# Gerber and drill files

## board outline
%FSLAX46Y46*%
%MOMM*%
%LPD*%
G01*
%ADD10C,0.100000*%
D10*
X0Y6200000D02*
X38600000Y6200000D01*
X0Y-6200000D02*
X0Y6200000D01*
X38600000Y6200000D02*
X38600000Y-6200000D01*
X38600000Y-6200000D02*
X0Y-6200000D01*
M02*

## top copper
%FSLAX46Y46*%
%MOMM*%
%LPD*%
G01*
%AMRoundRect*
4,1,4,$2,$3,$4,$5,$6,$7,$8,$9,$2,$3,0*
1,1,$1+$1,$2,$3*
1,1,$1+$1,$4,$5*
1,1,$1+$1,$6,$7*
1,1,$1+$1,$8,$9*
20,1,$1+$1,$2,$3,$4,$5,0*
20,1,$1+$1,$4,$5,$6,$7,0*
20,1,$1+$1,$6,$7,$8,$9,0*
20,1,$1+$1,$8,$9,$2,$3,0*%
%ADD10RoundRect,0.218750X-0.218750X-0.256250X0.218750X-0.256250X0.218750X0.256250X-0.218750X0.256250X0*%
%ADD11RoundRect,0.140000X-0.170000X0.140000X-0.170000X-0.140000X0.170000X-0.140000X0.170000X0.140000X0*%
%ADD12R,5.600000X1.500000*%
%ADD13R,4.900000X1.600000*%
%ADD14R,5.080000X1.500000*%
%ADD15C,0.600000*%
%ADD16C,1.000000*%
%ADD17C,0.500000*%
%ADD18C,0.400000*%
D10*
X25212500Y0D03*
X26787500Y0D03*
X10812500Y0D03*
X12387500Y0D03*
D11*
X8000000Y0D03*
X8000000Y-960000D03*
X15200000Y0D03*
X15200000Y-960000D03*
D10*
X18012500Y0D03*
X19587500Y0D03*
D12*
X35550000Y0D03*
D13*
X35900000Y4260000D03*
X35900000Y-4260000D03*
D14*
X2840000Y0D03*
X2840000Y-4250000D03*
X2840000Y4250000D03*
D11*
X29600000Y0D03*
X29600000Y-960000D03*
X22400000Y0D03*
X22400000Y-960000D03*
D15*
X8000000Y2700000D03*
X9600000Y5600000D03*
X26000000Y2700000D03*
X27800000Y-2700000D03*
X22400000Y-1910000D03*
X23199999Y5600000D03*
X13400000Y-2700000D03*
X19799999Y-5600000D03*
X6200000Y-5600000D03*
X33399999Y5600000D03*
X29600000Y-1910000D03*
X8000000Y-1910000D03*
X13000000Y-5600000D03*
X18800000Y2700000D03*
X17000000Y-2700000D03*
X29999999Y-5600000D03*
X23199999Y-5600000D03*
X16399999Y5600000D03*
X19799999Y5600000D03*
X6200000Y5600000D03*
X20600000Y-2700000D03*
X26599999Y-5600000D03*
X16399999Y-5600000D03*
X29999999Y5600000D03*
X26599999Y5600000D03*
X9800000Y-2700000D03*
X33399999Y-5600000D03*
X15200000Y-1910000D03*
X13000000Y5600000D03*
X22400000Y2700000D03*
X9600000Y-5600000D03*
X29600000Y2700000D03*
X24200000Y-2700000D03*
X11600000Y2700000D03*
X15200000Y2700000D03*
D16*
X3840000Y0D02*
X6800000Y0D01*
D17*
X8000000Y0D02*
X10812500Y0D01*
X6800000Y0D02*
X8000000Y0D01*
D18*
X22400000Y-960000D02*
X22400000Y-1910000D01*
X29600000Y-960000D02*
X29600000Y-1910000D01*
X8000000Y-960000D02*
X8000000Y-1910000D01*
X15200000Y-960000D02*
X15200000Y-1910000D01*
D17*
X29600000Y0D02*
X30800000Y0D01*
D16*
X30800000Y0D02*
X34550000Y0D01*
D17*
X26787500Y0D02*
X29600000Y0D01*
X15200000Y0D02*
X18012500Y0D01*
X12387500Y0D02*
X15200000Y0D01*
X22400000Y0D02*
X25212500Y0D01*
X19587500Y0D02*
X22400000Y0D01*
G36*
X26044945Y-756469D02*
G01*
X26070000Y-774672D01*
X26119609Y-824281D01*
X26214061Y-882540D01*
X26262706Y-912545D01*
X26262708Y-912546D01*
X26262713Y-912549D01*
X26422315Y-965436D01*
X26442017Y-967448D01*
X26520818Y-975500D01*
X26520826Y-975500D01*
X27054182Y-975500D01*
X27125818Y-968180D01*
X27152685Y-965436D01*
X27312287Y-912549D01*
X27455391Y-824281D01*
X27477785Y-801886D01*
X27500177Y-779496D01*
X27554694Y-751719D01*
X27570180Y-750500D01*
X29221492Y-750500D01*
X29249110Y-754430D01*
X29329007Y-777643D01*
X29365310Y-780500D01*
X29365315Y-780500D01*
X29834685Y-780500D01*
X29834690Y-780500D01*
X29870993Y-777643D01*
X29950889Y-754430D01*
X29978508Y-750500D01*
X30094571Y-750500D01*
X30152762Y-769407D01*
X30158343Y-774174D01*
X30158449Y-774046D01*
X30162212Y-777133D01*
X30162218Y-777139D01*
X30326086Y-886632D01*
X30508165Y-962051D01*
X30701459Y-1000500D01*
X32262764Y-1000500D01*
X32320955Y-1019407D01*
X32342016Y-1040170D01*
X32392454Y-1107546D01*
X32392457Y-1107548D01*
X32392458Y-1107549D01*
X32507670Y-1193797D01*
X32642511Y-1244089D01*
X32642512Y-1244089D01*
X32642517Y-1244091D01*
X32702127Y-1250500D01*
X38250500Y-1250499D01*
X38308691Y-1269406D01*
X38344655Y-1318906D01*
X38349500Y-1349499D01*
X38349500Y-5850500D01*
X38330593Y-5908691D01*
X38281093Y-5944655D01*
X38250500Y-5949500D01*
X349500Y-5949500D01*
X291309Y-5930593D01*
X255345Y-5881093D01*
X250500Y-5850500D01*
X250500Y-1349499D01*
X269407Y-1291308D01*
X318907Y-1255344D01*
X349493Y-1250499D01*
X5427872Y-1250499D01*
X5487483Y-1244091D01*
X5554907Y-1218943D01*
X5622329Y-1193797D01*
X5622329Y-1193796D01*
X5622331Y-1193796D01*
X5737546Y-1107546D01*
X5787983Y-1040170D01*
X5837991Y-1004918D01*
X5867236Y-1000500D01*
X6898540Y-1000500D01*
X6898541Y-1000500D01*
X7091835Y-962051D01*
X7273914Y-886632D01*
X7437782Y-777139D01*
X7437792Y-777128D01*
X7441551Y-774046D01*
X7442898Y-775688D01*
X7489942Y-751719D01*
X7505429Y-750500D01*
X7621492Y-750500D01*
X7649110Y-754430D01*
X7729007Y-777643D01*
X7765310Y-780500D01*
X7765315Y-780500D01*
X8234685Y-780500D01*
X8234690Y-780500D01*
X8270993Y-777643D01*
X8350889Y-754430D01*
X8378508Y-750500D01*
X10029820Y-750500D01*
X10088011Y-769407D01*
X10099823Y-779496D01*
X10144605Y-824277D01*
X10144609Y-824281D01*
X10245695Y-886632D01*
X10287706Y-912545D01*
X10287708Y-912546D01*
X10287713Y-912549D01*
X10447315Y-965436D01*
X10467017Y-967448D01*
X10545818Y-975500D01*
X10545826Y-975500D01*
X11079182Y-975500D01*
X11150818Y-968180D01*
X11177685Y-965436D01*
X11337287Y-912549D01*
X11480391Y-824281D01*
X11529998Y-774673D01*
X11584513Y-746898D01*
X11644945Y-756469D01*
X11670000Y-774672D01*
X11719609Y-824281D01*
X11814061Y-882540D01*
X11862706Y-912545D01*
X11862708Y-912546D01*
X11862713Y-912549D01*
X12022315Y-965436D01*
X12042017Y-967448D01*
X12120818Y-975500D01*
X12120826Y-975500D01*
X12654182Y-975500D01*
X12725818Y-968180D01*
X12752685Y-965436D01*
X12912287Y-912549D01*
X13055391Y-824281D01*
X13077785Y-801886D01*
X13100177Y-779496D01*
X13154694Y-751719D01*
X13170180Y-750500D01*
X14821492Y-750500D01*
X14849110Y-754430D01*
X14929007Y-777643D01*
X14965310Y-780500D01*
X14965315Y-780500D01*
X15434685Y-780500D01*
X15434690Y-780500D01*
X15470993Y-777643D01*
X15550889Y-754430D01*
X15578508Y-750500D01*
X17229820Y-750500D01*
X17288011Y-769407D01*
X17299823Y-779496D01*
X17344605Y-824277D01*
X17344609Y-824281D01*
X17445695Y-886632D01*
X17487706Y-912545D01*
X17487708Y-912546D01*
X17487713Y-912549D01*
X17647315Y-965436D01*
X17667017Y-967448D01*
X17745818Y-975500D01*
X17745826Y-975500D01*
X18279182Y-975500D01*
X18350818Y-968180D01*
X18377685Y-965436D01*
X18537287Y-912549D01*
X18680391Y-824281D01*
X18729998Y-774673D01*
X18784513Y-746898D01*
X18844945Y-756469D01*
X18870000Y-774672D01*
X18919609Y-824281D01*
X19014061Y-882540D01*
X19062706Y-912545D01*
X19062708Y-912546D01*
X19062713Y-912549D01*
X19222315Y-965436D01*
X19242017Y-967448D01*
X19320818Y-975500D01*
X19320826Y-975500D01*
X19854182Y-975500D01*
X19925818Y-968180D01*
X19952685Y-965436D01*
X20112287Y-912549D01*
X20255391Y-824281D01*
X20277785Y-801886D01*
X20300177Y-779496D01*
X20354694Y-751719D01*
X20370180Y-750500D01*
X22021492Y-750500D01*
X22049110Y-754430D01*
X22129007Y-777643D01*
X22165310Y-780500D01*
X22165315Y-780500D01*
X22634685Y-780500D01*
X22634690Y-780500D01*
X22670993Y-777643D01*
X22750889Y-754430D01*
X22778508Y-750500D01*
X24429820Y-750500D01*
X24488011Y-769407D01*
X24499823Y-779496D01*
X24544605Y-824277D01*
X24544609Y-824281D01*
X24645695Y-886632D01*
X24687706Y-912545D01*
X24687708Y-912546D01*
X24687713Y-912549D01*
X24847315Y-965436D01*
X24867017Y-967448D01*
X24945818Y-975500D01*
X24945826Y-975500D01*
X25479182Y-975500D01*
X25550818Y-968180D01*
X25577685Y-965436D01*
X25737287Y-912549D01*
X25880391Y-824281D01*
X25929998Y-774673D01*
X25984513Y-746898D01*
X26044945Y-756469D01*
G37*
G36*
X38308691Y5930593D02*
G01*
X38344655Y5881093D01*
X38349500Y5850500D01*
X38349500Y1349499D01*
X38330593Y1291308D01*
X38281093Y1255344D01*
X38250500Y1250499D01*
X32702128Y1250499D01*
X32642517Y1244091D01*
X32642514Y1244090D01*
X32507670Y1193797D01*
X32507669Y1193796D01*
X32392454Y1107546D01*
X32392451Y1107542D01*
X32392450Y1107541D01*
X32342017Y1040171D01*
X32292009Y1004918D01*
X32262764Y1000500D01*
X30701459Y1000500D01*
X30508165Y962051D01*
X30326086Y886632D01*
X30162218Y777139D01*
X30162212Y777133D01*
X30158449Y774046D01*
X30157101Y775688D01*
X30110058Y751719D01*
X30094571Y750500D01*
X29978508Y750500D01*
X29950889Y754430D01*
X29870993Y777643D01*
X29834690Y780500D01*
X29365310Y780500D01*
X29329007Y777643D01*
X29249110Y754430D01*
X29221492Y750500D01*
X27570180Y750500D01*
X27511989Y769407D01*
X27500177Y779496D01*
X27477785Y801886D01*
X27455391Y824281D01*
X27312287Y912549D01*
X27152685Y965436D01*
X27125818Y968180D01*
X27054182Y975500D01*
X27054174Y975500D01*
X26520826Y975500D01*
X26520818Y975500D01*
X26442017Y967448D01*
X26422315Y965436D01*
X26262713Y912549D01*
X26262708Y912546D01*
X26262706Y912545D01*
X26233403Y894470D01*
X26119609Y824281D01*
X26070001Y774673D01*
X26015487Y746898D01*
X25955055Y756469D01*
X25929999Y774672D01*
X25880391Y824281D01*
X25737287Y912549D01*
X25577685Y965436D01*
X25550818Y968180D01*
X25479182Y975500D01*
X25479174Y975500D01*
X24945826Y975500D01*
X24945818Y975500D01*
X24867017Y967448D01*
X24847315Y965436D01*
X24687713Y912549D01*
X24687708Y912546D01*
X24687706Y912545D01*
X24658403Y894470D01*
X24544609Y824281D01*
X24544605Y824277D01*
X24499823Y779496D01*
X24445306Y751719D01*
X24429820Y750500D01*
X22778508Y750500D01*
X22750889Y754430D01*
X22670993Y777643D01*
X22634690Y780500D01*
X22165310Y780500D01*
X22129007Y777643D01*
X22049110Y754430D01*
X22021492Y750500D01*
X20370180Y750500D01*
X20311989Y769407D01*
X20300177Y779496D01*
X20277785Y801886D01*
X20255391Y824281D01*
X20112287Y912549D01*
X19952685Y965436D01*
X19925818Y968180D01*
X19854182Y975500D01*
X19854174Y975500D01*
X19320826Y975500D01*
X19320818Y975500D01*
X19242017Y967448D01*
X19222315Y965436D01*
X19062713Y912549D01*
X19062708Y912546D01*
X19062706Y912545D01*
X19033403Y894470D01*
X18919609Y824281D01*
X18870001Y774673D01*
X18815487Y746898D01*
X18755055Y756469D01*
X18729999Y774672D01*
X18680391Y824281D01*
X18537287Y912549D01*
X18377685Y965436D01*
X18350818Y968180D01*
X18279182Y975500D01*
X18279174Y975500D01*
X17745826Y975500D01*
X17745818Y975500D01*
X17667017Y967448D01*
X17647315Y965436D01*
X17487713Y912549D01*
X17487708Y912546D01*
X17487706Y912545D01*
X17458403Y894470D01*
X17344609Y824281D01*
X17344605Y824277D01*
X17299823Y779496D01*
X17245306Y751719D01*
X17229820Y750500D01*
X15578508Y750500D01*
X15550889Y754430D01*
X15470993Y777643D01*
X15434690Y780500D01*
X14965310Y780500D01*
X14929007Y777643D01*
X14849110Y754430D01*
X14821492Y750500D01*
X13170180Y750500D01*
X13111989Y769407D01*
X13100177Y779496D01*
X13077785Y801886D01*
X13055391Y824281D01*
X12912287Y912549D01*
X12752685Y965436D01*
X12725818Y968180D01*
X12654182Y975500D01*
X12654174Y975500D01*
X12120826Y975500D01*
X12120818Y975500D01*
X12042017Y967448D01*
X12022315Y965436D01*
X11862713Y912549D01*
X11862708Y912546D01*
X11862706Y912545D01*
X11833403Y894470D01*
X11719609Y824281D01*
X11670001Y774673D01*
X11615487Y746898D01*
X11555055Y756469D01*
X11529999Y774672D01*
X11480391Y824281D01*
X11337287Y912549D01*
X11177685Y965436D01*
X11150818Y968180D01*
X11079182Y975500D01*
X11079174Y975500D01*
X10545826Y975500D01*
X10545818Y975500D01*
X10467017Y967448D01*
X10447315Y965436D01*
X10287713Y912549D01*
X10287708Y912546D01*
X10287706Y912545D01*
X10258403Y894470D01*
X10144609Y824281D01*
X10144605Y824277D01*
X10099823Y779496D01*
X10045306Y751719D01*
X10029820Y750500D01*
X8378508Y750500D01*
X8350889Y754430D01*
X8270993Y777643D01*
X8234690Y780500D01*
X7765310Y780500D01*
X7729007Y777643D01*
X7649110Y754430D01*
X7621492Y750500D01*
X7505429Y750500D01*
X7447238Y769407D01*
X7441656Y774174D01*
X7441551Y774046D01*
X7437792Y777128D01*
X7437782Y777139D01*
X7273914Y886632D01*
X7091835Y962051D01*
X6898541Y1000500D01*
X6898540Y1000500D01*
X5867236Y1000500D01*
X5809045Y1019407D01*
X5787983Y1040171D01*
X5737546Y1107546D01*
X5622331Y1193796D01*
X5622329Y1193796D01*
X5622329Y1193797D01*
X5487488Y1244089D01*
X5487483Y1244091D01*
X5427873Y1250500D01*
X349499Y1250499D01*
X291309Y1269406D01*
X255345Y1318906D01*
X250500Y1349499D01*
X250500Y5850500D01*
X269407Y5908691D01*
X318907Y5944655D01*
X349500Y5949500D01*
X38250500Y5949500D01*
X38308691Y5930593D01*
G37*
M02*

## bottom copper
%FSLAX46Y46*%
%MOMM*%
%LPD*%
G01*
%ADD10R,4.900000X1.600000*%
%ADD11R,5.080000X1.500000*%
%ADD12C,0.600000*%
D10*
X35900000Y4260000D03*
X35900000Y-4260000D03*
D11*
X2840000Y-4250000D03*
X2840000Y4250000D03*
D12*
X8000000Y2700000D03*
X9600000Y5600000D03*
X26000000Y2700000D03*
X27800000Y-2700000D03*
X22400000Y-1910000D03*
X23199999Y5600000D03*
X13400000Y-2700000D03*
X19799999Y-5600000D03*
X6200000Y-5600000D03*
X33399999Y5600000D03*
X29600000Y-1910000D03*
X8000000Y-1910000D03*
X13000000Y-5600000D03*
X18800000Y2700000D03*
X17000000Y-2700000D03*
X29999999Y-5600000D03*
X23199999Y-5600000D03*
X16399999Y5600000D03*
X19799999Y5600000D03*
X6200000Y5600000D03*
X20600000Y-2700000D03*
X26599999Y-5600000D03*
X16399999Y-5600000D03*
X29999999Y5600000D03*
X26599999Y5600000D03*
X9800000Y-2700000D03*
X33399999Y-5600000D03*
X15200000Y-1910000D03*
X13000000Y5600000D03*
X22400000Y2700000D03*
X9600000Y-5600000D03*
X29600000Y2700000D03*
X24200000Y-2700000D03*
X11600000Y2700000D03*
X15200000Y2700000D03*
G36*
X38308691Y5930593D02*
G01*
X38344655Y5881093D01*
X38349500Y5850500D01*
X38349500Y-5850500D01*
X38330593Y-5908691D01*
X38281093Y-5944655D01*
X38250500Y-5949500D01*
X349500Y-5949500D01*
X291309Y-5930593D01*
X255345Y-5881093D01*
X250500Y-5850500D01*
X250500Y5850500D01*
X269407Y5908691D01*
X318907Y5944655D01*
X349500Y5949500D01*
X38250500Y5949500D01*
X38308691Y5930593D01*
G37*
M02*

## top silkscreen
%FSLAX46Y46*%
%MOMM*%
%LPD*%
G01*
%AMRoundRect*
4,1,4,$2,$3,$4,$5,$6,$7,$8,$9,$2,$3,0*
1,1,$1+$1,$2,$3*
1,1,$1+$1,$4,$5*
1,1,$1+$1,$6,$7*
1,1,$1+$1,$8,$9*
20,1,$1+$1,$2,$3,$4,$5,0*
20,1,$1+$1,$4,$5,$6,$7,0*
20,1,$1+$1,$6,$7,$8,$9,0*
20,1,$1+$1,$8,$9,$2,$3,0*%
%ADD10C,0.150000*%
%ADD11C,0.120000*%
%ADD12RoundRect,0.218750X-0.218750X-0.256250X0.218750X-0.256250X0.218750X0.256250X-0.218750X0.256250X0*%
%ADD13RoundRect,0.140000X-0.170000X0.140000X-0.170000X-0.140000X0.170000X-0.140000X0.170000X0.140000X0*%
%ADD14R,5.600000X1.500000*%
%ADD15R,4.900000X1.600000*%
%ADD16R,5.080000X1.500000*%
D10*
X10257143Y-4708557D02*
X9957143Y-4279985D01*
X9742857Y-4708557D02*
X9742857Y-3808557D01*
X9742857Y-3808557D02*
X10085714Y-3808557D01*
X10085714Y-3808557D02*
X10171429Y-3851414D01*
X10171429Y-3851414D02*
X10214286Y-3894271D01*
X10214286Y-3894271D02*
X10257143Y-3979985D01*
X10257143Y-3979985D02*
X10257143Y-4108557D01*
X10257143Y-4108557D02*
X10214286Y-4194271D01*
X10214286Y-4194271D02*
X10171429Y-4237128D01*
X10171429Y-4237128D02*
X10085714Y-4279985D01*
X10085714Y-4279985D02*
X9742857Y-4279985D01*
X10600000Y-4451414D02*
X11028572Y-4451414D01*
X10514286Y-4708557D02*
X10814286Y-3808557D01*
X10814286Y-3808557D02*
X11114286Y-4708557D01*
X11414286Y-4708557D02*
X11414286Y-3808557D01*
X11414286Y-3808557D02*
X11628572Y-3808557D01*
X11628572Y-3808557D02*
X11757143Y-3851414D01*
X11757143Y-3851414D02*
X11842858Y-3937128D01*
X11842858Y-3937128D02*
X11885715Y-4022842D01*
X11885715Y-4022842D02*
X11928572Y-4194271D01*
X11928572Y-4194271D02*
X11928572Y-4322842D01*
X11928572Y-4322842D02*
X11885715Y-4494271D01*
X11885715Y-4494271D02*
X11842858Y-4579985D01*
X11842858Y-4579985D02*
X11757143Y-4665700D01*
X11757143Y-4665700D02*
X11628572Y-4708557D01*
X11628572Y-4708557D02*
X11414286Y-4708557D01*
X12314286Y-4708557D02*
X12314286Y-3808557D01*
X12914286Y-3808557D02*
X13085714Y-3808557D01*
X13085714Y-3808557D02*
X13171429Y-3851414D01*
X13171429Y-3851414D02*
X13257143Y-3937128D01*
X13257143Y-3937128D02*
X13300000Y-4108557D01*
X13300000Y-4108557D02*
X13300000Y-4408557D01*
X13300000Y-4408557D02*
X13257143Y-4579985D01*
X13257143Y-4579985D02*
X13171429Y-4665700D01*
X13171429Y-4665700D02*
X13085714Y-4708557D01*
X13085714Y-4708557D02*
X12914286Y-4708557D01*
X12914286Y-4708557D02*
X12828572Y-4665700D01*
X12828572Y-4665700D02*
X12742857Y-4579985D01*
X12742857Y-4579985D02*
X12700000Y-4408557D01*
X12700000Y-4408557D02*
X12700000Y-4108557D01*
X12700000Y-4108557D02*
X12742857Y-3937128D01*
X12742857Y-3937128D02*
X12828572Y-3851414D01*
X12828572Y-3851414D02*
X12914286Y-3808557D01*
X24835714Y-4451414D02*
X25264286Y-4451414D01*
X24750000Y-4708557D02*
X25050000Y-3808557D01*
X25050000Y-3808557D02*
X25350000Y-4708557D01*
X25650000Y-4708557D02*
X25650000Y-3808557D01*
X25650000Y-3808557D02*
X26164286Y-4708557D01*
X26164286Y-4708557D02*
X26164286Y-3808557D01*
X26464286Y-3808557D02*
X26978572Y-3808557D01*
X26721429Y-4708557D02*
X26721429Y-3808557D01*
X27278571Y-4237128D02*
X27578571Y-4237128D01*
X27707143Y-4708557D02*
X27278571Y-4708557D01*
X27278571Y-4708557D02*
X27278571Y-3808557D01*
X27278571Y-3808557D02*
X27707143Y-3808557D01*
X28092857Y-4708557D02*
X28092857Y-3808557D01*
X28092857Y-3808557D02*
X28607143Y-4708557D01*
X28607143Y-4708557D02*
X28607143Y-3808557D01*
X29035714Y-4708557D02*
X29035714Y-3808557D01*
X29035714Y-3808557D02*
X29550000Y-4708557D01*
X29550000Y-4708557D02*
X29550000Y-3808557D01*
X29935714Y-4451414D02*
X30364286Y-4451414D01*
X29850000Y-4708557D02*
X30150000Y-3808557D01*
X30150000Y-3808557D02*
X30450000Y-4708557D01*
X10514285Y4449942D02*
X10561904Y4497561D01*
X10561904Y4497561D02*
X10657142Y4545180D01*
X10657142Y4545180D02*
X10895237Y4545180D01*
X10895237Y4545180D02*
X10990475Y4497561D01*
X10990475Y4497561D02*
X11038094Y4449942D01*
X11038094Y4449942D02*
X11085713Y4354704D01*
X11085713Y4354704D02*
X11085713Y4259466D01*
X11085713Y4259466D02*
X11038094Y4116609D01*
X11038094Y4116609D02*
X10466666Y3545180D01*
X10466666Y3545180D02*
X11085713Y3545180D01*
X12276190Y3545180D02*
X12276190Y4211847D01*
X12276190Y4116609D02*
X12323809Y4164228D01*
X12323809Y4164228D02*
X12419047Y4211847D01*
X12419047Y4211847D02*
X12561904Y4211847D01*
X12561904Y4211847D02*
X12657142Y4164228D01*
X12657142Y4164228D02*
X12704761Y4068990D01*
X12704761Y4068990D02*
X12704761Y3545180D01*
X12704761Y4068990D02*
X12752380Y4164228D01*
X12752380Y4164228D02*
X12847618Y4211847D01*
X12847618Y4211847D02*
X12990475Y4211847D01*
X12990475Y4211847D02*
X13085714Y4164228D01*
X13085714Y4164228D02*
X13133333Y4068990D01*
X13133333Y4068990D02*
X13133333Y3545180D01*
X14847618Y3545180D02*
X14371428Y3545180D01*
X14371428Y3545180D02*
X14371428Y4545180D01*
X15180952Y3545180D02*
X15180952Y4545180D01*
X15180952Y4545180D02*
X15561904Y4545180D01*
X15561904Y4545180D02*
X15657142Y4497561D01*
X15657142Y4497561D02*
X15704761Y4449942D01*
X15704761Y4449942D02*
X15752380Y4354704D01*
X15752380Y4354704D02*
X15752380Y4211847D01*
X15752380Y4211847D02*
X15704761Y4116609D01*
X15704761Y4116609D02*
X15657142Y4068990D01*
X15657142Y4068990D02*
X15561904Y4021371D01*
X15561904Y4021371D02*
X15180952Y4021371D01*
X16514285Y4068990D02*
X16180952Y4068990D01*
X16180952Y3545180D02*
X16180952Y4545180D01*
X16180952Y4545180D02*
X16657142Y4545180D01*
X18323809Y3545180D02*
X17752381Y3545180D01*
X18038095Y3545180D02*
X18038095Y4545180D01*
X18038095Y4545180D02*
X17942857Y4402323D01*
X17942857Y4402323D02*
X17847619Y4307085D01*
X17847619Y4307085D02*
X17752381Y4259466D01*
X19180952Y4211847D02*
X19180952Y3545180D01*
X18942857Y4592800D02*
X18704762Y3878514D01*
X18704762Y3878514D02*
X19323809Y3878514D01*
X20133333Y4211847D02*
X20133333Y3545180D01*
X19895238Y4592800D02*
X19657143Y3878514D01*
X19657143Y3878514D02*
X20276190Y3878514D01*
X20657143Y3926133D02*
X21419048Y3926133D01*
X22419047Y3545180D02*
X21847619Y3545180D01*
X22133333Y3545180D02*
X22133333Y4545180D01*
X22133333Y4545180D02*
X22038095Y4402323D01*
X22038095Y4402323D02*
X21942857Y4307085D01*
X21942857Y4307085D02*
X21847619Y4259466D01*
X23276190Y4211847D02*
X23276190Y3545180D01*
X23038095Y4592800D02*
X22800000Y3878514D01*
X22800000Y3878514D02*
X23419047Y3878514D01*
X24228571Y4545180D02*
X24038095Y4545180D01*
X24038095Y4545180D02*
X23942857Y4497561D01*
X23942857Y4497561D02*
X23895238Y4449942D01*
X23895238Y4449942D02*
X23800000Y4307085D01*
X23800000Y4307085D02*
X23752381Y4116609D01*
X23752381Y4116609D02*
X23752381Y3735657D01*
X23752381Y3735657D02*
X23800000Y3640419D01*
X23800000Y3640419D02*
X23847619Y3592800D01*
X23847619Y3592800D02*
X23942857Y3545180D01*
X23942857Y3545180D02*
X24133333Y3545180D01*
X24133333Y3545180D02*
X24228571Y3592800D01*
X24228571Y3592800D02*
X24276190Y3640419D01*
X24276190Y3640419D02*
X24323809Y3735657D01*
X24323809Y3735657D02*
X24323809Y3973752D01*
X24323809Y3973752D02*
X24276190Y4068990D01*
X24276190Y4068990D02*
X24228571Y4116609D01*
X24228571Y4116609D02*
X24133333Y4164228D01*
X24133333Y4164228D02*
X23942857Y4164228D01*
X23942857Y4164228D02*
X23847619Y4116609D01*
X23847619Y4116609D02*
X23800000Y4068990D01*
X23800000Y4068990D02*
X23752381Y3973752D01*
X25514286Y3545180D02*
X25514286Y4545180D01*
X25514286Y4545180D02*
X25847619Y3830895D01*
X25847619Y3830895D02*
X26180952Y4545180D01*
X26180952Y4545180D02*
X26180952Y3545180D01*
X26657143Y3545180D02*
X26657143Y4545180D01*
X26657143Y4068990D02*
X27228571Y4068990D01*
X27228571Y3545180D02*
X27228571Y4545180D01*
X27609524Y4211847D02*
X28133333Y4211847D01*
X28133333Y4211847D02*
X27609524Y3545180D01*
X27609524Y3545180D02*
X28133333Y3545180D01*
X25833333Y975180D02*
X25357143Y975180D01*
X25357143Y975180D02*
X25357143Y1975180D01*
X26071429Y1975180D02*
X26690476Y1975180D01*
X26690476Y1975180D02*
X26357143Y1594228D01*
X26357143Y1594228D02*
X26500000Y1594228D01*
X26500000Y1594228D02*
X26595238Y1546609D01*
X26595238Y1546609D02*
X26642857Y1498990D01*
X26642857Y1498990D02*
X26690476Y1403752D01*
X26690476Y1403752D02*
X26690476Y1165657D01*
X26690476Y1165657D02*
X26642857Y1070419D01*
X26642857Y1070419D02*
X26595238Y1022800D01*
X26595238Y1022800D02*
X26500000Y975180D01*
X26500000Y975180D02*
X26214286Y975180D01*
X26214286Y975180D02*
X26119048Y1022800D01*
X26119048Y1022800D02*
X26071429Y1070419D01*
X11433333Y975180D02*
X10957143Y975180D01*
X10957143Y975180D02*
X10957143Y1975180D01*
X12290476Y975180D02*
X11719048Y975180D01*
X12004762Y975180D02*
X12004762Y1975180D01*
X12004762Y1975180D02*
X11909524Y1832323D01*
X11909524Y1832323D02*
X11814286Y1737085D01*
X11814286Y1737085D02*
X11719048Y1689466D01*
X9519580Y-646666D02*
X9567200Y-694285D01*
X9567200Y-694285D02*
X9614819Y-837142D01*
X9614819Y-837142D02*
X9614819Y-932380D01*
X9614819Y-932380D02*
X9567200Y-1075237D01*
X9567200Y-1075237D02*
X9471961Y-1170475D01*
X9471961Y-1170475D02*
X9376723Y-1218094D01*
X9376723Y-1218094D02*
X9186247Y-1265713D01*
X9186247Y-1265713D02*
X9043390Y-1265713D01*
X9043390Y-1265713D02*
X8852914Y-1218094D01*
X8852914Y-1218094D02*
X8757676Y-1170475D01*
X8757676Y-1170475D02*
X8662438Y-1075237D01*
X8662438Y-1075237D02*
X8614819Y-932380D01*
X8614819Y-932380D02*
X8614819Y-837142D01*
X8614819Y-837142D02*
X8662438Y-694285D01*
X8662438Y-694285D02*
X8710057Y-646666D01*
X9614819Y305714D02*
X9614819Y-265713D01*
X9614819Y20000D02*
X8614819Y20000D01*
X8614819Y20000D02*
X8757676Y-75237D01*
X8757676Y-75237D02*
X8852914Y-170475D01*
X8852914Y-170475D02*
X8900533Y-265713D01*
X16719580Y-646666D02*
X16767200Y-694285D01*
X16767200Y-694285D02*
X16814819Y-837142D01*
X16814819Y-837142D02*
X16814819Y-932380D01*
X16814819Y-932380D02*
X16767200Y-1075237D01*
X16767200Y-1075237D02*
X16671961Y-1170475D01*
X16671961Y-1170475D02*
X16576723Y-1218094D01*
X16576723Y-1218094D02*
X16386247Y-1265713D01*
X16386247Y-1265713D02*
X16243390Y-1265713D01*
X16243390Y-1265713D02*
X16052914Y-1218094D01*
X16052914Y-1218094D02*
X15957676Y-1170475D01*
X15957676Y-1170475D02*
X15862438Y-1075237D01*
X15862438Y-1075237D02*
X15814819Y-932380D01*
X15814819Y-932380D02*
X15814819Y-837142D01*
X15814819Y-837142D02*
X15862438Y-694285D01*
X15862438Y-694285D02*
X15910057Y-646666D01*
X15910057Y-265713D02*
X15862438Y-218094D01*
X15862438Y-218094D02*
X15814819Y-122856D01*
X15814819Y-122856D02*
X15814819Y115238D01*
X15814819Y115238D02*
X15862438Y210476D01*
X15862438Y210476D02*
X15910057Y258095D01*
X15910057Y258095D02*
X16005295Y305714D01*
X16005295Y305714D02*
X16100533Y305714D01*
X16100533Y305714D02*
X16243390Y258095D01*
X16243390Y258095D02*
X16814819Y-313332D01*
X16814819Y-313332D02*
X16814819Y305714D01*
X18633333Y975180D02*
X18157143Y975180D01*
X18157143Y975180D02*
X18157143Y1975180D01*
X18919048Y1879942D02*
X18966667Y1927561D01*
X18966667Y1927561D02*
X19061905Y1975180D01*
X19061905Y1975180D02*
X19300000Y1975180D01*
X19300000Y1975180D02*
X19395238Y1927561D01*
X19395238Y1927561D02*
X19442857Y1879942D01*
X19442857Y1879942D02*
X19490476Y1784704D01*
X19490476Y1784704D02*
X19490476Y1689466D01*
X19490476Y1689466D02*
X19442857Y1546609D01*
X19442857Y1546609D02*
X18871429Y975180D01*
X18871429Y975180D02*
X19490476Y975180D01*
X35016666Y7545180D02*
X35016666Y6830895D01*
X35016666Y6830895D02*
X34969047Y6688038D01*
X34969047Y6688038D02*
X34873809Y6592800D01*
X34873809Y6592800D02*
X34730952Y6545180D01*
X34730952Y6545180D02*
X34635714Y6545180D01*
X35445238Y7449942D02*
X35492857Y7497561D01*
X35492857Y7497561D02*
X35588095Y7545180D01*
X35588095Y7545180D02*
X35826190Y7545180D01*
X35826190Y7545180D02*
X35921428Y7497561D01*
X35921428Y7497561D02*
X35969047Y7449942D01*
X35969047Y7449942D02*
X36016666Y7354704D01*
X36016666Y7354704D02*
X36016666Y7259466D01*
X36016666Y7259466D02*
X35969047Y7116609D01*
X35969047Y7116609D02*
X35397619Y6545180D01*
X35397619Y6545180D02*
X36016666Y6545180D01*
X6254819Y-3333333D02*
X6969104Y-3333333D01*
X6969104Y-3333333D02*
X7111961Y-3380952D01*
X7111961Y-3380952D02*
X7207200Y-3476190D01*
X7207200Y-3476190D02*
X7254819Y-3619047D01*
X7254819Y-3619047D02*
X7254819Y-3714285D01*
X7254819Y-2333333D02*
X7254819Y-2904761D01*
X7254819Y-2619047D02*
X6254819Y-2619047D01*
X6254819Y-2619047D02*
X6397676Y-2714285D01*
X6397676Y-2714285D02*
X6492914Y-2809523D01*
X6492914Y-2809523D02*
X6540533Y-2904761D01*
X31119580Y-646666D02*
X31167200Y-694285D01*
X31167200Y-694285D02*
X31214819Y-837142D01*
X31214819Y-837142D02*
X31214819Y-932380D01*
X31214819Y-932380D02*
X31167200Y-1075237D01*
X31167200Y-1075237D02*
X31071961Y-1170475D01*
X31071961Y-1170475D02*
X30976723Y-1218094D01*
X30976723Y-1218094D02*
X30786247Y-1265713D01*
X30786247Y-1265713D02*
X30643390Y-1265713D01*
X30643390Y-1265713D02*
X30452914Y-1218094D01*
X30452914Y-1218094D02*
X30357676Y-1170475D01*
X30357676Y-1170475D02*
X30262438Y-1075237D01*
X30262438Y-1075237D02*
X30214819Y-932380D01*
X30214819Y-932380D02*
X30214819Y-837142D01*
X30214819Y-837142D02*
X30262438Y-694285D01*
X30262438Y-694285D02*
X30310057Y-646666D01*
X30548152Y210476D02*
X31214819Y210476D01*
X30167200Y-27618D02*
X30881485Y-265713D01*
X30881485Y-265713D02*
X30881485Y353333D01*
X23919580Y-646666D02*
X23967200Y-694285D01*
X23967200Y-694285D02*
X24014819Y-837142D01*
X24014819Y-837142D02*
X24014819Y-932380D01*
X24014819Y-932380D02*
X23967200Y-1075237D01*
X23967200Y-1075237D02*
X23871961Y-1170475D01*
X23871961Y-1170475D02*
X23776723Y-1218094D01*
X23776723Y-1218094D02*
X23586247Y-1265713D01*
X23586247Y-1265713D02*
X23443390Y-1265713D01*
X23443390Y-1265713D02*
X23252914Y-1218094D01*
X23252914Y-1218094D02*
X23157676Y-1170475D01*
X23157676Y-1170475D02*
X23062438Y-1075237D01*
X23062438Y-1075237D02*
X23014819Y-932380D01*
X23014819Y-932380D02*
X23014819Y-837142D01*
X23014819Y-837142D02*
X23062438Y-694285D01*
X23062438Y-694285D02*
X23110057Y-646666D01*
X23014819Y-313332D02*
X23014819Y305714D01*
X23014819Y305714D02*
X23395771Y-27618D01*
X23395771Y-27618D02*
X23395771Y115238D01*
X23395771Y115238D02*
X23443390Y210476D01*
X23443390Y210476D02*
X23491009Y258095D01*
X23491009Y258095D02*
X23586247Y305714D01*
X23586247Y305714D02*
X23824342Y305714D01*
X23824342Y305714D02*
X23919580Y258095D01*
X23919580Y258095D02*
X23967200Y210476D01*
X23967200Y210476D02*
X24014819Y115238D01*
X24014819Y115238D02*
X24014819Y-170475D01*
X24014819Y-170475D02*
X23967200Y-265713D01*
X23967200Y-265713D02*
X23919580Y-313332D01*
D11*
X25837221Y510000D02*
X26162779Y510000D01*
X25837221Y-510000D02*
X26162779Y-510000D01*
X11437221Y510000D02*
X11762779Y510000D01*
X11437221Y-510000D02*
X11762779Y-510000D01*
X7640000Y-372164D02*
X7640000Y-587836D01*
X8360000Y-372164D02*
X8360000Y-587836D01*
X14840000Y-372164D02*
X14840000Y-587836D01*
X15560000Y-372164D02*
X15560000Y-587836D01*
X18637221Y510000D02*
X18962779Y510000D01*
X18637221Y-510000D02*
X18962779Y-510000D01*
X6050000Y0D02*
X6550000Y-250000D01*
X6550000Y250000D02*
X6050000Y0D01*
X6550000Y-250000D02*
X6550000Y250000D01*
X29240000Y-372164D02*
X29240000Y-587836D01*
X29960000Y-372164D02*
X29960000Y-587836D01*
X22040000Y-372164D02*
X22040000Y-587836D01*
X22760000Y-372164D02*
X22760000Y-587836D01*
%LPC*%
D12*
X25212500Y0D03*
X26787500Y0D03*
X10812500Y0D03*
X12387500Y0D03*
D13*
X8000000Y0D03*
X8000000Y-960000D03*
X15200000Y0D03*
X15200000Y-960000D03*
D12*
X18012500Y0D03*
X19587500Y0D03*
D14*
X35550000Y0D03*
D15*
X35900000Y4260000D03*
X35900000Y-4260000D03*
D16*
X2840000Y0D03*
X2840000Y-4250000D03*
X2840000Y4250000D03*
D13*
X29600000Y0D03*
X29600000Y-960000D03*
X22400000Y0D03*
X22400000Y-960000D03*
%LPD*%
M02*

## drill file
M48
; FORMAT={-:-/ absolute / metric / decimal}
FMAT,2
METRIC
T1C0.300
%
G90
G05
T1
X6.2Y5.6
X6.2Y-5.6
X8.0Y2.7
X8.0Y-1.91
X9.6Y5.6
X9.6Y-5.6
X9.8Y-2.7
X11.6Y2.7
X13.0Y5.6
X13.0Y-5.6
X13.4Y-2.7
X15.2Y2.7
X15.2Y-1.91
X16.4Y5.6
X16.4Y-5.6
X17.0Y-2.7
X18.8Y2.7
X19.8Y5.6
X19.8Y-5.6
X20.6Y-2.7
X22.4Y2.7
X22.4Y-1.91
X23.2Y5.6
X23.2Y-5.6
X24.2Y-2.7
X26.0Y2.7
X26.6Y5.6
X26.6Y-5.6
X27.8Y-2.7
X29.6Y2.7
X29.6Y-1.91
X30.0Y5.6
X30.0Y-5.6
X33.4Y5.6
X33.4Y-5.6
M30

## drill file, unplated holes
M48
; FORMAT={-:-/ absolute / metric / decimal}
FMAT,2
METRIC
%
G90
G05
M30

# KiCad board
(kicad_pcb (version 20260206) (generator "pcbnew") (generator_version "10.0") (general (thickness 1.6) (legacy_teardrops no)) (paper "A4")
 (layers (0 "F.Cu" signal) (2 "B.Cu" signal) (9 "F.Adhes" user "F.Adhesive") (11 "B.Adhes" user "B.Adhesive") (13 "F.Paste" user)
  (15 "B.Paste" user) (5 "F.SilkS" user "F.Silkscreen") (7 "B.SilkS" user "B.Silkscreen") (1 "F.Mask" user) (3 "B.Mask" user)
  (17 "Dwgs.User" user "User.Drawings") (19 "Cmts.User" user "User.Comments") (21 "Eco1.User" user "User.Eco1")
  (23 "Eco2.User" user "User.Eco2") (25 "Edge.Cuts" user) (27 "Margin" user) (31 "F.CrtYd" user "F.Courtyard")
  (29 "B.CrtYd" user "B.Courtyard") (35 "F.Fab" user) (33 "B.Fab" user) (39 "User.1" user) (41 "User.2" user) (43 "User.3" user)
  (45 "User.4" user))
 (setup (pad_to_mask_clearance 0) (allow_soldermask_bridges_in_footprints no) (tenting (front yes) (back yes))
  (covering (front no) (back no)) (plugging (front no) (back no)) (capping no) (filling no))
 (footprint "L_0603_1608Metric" (layer "F.Cu") (at 26 0)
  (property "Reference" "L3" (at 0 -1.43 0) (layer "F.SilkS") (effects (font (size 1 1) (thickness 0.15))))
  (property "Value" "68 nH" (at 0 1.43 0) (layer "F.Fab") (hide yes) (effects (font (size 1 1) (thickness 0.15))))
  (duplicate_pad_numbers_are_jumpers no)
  (fp_line (start -0.162779 -0.51) (end 0.162779 -0.51) (stroke (width 0.12) (type solid)) (layer "F.SilkS"))
  (fp_line (start -0.162779 0.51) (end 0.162779 0.51) (stroke (width 0.12) (type solid)) (layer "F.SilkS"))
  (pad "1" smd roundrect (at -0.7875 0) (size 0.875 0.95) (layers "F.Cu" "F.Mask" "F.Paste") (roundrect_rratio 0.25) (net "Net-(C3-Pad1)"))
  (pad "2" smd roundrect (at 0.7875 0) (size 0.875 0.95) (layers "F.Cu" "F.Mask" "F.Paste") (roundrect_rratio 0.25) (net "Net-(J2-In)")))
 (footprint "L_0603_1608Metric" (layer "F.Cu") (at 11.6 0)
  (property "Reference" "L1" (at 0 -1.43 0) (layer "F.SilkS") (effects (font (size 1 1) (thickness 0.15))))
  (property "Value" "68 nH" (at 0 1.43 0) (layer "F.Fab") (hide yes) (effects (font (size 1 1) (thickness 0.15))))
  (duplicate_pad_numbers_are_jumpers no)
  (fp_line (start -0.162779 -0.51) (end 0.162779 -0.51) (stroke (width 0.12) (type solid)) (layer "F.SilkS"))
  (fp_line (start -0.162779 0.51) (end 0.162779 0.51) (stroke (width 0.12) (type solid)) (layer "F.SilkS"))
  (pad "1" smd roundrect (at -0.7875 0) (size 0.875 0.95) (layers "F.Cu" "F.Mask" "F.Paste") (roundrect_rratio 0.25) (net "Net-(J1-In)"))
  (pad "2" smd roundrect (at 0.7875 0) (size 0.875 0.95) (layers "F.Cu" "F.Mask" "F.Paste") (roundrect_rratio 0.25) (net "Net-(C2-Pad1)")))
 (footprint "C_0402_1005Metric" (layer "F.Cu") (at 8 0.48 -90)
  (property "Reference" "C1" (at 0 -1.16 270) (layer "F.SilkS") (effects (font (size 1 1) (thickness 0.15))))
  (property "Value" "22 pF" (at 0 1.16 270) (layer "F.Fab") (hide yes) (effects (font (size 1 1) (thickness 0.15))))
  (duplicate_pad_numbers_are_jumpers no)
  (fp_line (start -0.107836 0.36) (end 0.107836 0.36) (stroke (width 0.12) (type solid)) (layer "F.SilkS"))
  (fp_line (start -0.107836 -0.36) (end 0.107836 -0.36) (stroke (width 0.12) (type solid)) (layer "F.SilkS"))
  (pad "1" smd roundrect (at -0.48 0 270) (size 0.56 0.62) (layers "F.Cu" "F.Mask" "F.Paste") (roundrect_rratio 0.25) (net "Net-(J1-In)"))
  (pad "2" smd roundrect (at 0.48 0 270) (size 0.56 0.62) (layers "F.Cu" "F.Mask" "F.Paste") (roundrect_rratio 0.25) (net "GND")
   (zone_connect 2)))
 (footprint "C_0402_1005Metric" (layer "F.Cu") (at 15.2 0.48 -90)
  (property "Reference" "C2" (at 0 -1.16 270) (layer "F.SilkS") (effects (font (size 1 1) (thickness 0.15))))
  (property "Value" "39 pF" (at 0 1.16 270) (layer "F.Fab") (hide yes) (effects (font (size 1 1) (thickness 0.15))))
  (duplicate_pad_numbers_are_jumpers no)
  (fp_line (start -0.107836 0.36) (end 0.107836 0.36) (stroke (width 0.12) (type solid)) (layer "F.SilkS"))
  (fp_line (start -0.107836 -0.36) (end 0.107836 -0.36) (stroke (width 0.12) (type solid)) (layer "F.SilkS"))
  (pad "1" smd roundrect (at -0.48 0 270) (size 0.56 0.62) (layers "F.Cu" "F.Mask" "F.Paste") (roundrect_rratio 0.25) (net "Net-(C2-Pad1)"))
  (pad "2" smd roundrect (at 0.48 0 270) (size 0.56 0.62) (layers "F.Cu" "F.Mask" "F.Paste") (roundrect_rratio 0.25) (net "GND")
   (zone_connect 2)))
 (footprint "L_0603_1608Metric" (layer "F.Cu") (at 18.8 0)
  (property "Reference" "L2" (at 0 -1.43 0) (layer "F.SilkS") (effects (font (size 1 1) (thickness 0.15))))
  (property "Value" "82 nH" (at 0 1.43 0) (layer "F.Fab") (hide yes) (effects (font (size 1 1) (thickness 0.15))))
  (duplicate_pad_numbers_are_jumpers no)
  (fp_line (start -0.162779 -0.51) (end 0.162779 -0.51) (stroke (width 0.12) (type solid)) (layer "F.SilkS"))
  (fp_line (start -0.162779 0.51) (end 0.162779 0.51) (stroke (width 0.12) (type solid)) (layer "F.SilkS"))
  (pad "1" smd roundrect (at -0.7875 0) (size 0.875 0.95) (layers "F.Cu" "F.Mask" "F.Paste") (roundrect_rratio 0.25) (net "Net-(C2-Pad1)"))
  (pad "2" smd roundrect (at 0.7875 0) (size 0.875 0.95) (layers "F.Cu" "F.Mask" "F.Paste") (roundrect_rratio 0.25) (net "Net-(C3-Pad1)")))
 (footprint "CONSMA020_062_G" (layer "F.Cu") (at 38.35 0)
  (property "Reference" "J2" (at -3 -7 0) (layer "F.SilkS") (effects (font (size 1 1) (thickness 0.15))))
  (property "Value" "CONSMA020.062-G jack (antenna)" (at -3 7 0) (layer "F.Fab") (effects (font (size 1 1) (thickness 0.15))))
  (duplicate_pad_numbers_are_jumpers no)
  (pad "1" smd rect (at -2.8 0) (size 5.6 1.5) (layers "F.Cu" "F.Mask" "F.Paste") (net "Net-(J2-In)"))
  (pad "2" smd rect (at -2.45 -4.26) (size 4.9 1.6) (layers "F.Cu" "F.Mask" "F.Paste") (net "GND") (zone_connect 2))
  (pad "2" smd rect (at -2.45 -4.26) (size 4.9 1.6) (layers "B.Cu" "B.Mask" "B.Paste") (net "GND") (zone_connect 2))
  (pad "2" smd rect (at -2.45 4.26) (size 4.9 1.6) (layers "F.Cu" "F.Mask" "F.Paste") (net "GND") (zone_connect 2))
  (pad "2" smd rect (at -2.45 4.26) (size 4.9 1.6) (layers "B.Cu" "B.Mask" "B.Paste") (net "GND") (zone_connect 2)))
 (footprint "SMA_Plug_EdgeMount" (layer "F.Cu") (at 2.84 0 180)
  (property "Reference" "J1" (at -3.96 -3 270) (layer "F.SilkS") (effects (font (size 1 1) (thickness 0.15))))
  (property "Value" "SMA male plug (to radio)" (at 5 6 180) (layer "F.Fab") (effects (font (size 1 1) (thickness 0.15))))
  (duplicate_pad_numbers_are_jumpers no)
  (fp_line (start -3.21 0) (end -3.71 -0.25) (stroke (width 0.12) (type solid)) (layer "F.SilkS"))
  (fp_line (start -3.71 0.25) (end -3.21 0) (stroke (width 0.12) (type solid)) (layer "F.SilkS"))
  (fp_line (start -3.71 -0.25) (end -3.71 0.25) (stroke (width 0.12) (type solid)) (layer "F.SilkS"))
  (pad "1" smd rect (at 0 0 270) (size 1.5 5.08) (layers "F.Cu" "F.Mask" "F.Paste") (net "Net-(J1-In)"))
  (pad "2" smd rect (at 0 -4.25 270) (size 1.5 5.08) (layers "F.Cu" "F.Mask" "F.Paste") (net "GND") (zone_connect 2))
  (pad "2" smd rect (at 0 -4.25 270) (size 1.5 5.08) (layers "B.Cu" "B.Mask" "B.Paste") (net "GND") (zone_connect 2))
  (pad "2" smd rect (at 0 4.25 270) (size 1.5 5.08) (layers "F.Cu" "F.Mask" "F.Paste") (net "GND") (zone_connect 2))
  (pad "2" smd rect (at 0 4.25 270) (size 1.5 5.08) (layers "B.Cu" "B.Mask" "B.Paste") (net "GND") (zone_connect 2)))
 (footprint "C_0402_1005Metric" (layer "F.Cu") (at 29.6 0.48 -90)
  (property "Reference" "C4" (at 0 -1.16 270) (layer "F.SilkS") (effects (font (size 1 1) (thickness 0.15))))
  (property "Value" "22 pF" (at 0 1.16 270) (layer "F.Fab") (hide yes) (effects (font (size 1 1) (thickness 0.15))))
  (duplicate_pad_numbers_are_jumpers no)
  (fp_line (start -0.107836 0.36) (end 0.107836 0.36) (stroke (width 0.12) (type solid)) (layer "F.SilkS"))
  (fp_line (start -0.107836 -0.36) (end 0.107836 -0.36) (stroke (width 0.12) (type solid)) (layer "F.SilkS"))
  (pad "1" smd roundrect (at -0.48 0 270) (size 0.56 0.62) (layers "F.Cu" "F.Mask" "F.Paste") (roundrect_rratio 0.25) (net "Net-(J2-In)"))
  (pad "2" smd roundrect (at 0.48 0 270) (size 0.56 0.62) (layers "F.Cu" "F.Mask" "F.Paste") (roundrect_rratio 0.25) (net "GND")
   (zone_connect 2)))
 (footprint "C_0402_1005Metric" (layer "F.Cu") (at 22.4 0.48 -90)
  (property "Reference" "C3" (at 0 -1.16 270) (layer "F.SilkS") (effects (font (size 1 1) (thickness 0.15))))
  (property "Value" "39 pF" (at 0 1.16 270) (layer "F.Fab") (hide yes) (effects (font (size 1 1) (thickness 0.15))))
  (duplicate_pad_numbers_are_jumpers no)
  (fp_line (start -0.107836 0.36) (end 0.107836 0.36) (stroke (width 0.12) (type solid)) (layer "F.SilkS"))
  (fp_line (start -0.107836 -0.36) (end 0.107836 -0.36) (stroke (width 0.12) (type solid)) (layer "F.SilkS"))
  (pad "1" smd roundrect (at -0.48 0 270) (size 0.56 0.62) (layers "F.Cu" "F.Mask" "F.Paste") (roundrect_rratio 0.25) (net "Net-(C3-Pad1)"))
  (pad "2" smd roundrect (at 0.48 0 270) (size 0.56 0.62) (layers "F.Cu" "F.Mask" "F.Paste") (roundrect_rratio 0.25) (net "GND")
   (zone_connect 2)))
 (gr_line (start 0 -6.2) (end 38.6 -6.2) (stroke (width 0.1) (type default)) (layer "Edge.Cuts"))
 (gr_line (start 0 6.2) (end 0 -6.2) (stroke (width 0.1) (type default)) (layer "Edge.Cuts"))
 (gr_line (start 38.6 -6.2) (end 38.6 6.2) (stroke (width 0.1) (type default)) (layer "Edge.Cuts"))
 (gr_line (start 38.6 6.2) (end 0 6.2) (stroke (width 0.1) (type default)) (layer "Edge.Cuts"))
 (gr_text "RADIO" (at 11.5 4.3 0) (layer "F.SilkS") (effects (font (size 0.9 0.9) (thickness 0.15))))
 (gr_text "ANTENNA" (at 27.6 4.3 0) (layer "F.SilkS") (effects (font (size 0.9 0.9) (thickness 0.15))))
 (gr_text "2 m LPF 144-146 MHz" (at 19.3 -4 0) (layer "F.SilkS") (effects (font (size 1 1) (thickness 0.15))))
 (segment (start 3.84 0) (end 6.8 0) (width 1) (layer "F.Cu") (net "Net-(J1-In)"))
 (segment (start 8 0) (end 10.8125 0) (width 0.5) (layer "F.Cu") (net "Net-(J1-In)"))
 (segment (start 6.8 0) (end 8 0) (width 0.5) (layer "F.Cu") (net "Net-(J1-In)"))
 (segment (start 22.4 0.96) (end 22.4 1.91) (width 0.4) (layer "F.Cu") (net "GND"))
 (segment (start 29.6 0.96) (end 29.6 1.91) (width 0.4) (layer "F.Cu") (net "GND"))
 (segment (start 8 0.96) (end 8 1.91) (width 0.4) (layer "F.Cu") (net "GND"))
 (segment (start 15.2 0.96) (end 15.2 1.91) (width 0.4) (layer "F.Cu") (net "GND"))
 (via (at 8 -2.7) (size 0.6) (drill 0.3) (layers "F.Cu" "B.Cu") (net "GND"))
 (via (at 9.6 -5.6) (size 0.6) (drill 0.3) (layers "F.Cu" "B.Cu") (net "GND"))
 (via (at 26 -2.7) (size 0.6) (drill 0.3) (layers "F.Cu" "B.Cu") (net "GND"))
 (via (at 27.8 2.7) (size 0.6) (drill 0.3) (layers "F.Cu" "B.Cu") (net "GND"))
 (via (at 22.4 1.91) (size 0.6) (drill 0.3) (layers "F.Cu" "B.Cu") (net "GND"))
 (via (at 23.199999 -5.6) (size 0.6) (drill 0.3) (layers "F.Cu" "B.Cu") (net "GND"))
 (via (at 13.4 2.7) (size 0.6) (drill 0.3) (layers "F.Cu" "B.Cu") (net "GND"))
 (via (at 19.799999 5.6) (size 0.6) (drill 0.3) (layers "F.Cu" "B.Cu") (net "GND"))
 (via (at 6.2 5.6) (size 0.6) (drill 0.3) (layers "F.Cu" "B.Cu") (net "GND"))
 (via (at 33.399999 -5.6) (size 0.6) (drill 0.3) (layers "F.Cu" "B.Cu") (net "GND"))
 (via (at 29.6 1.91) (size 0.6) (drill 0.3) (layers "F.Cu" "B.Cu") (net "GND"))
 (via (at 8 1.91) (size 0.6) (drill 0.3) (layers "F.Cu" "B.Cu") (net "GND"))
 (via (at 13 5.6) (size 0.6) (drill 0.3) (layers "F.Cu" "B.Cu") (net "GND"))
 (via (at 18.8 -2.7) (size 0.6) (drill 0.3) (layers "F.Cu" "B.Cu") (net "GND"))
 (via (at 17 2.7) (size 0.6) (drill 0.3) (layers "F.Cu" "B.Cu") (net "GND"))
 (via (at 29.999999 5.6) (size 0.6) (drill 0.3) (layers "F.Cu" "B.Cu") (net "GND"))
 (via (at 23.199999 5.6) (size 0.6) (drill 0.3) (layers "F.Cu" "B.Cu") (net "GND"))
 (via (at 16.399999 -5.6) (size 0.6) (drill 0.3) (layers "F.Cu" "B.Cu") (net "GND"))
 (via (at 19.799999 -5.6) (size 0.6) (drill 0.3) (layers "F.Cu" "B.Cu") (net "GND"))
 (via (at 6.2 -5.6) (size 0.6) (drill 0.3) (layers "F.Cu" "B.Cu") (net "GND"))
 (via (at 20.6 2.7) (size 0.6) (drill 0.3) (layers "F.Cu" "B.Cu") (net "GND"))
 (via (at 26.599999 5.6) (size 0.6) (drill 0.3) (layers "F.Cu" "B.Cu") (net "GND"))
 (via (at 16.399999 5.6) (size 0.6) (drill 0.3) (layers "F.Cu" "B.Cu") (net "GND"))
 (via (at 29.999999 -5.6) (size 0.6) (drill 0.3) (layers "F.Cu" "B.Cu") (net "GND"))
 (via (at 26.599999 -5.6) (size 0.6) (drill 0.3) (layers "F.Cu" "B.Cu") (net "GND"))
 (via (at 9.8 2.7) (size 0.6) (drill 0.3) (layers "F.Cu" "B.Cu") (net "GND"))
 (via (at 33.399999 5.6) (size 0.6) (drill 0.3) (layers "F.Cu" "B.Cu") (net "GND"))
 (via (at 15.2 1.91) (size 0.6) (drill 0.3) (layers "F.Cu" "B.Cu") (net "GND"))
 (via (at 13 -5.6) (size 0.6) (drill 0.3) (layers "F.Cu" "B.Cu") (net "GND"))
 (via (at 22.4 -2.7) (size 0.6) (drill 0.3) (layers "F.Cu" "B.Cu") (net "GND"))
 (via (at 9.6 5.6) (size 0.6) (drill 0.3) (layers "F.Cu" "B.Cu") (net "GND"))
 (via (at 29.6 -2.7) (size 0.6) (drill 0.3) (layers "F.Cu" "B.Cu") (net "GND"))
 (via (at 24.2 2.7) (size 0.6) (drill 0.3) (layers "F.Cu" "B.Cu") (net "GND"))
 (via (at 11.6 -2.7) (size 0.6) (drill 0.3) (layers "F.Cu" "B.Cu") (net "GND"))
 (via (at 15.2 -2.7) (size 0.6) (drill 0.3) (layers "F.Cu" "B.Cu") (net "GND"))
 (segment (start 29.6 0) (end 30.8 0) (width 0.5) (layer "F.Cu") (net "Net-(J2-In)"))
 (segment (start 30.8 0) (end 34.55 0) (width 1) (layer "F.Cu") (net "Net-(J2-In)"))
 (segment (start 26.7875 0) (end 29.6 0) (width 0.5) (layer "F.Cu") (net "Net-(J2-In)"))
 (segment (start 15.2 0) (end 18.0125 0) (width 0.5) (layer "F.Cu") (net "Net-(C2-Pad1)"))
 (segment (start 12.3875 0) (end 15.2 0) (width 0.5) (layer "F.Cu") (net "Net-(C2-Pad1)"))
 (segment (start 22.4 0) (end 25.2125 0) (width 0.5) (layer "F.Cu") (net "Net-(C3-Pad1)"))
 (segment (start 19.5875 0) (end 22.4 0) (width 0.5) (layer "F.Cu") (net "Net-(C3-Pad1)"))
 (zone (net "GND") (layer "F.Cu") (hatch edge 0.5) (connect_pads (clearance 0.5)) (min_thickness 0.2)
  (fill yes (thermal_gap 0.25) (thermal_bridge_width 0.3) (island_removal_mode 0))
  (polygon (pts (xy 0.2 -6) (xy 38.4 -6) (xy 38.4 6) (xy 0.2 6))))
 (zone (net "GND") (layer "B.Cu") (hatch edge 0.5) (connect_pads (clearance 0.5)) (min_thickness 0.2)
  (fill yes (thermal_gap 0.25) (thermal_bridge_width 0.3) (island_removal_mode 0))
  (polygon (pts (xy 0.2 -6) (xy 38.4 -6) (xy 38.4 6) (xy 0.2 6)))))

